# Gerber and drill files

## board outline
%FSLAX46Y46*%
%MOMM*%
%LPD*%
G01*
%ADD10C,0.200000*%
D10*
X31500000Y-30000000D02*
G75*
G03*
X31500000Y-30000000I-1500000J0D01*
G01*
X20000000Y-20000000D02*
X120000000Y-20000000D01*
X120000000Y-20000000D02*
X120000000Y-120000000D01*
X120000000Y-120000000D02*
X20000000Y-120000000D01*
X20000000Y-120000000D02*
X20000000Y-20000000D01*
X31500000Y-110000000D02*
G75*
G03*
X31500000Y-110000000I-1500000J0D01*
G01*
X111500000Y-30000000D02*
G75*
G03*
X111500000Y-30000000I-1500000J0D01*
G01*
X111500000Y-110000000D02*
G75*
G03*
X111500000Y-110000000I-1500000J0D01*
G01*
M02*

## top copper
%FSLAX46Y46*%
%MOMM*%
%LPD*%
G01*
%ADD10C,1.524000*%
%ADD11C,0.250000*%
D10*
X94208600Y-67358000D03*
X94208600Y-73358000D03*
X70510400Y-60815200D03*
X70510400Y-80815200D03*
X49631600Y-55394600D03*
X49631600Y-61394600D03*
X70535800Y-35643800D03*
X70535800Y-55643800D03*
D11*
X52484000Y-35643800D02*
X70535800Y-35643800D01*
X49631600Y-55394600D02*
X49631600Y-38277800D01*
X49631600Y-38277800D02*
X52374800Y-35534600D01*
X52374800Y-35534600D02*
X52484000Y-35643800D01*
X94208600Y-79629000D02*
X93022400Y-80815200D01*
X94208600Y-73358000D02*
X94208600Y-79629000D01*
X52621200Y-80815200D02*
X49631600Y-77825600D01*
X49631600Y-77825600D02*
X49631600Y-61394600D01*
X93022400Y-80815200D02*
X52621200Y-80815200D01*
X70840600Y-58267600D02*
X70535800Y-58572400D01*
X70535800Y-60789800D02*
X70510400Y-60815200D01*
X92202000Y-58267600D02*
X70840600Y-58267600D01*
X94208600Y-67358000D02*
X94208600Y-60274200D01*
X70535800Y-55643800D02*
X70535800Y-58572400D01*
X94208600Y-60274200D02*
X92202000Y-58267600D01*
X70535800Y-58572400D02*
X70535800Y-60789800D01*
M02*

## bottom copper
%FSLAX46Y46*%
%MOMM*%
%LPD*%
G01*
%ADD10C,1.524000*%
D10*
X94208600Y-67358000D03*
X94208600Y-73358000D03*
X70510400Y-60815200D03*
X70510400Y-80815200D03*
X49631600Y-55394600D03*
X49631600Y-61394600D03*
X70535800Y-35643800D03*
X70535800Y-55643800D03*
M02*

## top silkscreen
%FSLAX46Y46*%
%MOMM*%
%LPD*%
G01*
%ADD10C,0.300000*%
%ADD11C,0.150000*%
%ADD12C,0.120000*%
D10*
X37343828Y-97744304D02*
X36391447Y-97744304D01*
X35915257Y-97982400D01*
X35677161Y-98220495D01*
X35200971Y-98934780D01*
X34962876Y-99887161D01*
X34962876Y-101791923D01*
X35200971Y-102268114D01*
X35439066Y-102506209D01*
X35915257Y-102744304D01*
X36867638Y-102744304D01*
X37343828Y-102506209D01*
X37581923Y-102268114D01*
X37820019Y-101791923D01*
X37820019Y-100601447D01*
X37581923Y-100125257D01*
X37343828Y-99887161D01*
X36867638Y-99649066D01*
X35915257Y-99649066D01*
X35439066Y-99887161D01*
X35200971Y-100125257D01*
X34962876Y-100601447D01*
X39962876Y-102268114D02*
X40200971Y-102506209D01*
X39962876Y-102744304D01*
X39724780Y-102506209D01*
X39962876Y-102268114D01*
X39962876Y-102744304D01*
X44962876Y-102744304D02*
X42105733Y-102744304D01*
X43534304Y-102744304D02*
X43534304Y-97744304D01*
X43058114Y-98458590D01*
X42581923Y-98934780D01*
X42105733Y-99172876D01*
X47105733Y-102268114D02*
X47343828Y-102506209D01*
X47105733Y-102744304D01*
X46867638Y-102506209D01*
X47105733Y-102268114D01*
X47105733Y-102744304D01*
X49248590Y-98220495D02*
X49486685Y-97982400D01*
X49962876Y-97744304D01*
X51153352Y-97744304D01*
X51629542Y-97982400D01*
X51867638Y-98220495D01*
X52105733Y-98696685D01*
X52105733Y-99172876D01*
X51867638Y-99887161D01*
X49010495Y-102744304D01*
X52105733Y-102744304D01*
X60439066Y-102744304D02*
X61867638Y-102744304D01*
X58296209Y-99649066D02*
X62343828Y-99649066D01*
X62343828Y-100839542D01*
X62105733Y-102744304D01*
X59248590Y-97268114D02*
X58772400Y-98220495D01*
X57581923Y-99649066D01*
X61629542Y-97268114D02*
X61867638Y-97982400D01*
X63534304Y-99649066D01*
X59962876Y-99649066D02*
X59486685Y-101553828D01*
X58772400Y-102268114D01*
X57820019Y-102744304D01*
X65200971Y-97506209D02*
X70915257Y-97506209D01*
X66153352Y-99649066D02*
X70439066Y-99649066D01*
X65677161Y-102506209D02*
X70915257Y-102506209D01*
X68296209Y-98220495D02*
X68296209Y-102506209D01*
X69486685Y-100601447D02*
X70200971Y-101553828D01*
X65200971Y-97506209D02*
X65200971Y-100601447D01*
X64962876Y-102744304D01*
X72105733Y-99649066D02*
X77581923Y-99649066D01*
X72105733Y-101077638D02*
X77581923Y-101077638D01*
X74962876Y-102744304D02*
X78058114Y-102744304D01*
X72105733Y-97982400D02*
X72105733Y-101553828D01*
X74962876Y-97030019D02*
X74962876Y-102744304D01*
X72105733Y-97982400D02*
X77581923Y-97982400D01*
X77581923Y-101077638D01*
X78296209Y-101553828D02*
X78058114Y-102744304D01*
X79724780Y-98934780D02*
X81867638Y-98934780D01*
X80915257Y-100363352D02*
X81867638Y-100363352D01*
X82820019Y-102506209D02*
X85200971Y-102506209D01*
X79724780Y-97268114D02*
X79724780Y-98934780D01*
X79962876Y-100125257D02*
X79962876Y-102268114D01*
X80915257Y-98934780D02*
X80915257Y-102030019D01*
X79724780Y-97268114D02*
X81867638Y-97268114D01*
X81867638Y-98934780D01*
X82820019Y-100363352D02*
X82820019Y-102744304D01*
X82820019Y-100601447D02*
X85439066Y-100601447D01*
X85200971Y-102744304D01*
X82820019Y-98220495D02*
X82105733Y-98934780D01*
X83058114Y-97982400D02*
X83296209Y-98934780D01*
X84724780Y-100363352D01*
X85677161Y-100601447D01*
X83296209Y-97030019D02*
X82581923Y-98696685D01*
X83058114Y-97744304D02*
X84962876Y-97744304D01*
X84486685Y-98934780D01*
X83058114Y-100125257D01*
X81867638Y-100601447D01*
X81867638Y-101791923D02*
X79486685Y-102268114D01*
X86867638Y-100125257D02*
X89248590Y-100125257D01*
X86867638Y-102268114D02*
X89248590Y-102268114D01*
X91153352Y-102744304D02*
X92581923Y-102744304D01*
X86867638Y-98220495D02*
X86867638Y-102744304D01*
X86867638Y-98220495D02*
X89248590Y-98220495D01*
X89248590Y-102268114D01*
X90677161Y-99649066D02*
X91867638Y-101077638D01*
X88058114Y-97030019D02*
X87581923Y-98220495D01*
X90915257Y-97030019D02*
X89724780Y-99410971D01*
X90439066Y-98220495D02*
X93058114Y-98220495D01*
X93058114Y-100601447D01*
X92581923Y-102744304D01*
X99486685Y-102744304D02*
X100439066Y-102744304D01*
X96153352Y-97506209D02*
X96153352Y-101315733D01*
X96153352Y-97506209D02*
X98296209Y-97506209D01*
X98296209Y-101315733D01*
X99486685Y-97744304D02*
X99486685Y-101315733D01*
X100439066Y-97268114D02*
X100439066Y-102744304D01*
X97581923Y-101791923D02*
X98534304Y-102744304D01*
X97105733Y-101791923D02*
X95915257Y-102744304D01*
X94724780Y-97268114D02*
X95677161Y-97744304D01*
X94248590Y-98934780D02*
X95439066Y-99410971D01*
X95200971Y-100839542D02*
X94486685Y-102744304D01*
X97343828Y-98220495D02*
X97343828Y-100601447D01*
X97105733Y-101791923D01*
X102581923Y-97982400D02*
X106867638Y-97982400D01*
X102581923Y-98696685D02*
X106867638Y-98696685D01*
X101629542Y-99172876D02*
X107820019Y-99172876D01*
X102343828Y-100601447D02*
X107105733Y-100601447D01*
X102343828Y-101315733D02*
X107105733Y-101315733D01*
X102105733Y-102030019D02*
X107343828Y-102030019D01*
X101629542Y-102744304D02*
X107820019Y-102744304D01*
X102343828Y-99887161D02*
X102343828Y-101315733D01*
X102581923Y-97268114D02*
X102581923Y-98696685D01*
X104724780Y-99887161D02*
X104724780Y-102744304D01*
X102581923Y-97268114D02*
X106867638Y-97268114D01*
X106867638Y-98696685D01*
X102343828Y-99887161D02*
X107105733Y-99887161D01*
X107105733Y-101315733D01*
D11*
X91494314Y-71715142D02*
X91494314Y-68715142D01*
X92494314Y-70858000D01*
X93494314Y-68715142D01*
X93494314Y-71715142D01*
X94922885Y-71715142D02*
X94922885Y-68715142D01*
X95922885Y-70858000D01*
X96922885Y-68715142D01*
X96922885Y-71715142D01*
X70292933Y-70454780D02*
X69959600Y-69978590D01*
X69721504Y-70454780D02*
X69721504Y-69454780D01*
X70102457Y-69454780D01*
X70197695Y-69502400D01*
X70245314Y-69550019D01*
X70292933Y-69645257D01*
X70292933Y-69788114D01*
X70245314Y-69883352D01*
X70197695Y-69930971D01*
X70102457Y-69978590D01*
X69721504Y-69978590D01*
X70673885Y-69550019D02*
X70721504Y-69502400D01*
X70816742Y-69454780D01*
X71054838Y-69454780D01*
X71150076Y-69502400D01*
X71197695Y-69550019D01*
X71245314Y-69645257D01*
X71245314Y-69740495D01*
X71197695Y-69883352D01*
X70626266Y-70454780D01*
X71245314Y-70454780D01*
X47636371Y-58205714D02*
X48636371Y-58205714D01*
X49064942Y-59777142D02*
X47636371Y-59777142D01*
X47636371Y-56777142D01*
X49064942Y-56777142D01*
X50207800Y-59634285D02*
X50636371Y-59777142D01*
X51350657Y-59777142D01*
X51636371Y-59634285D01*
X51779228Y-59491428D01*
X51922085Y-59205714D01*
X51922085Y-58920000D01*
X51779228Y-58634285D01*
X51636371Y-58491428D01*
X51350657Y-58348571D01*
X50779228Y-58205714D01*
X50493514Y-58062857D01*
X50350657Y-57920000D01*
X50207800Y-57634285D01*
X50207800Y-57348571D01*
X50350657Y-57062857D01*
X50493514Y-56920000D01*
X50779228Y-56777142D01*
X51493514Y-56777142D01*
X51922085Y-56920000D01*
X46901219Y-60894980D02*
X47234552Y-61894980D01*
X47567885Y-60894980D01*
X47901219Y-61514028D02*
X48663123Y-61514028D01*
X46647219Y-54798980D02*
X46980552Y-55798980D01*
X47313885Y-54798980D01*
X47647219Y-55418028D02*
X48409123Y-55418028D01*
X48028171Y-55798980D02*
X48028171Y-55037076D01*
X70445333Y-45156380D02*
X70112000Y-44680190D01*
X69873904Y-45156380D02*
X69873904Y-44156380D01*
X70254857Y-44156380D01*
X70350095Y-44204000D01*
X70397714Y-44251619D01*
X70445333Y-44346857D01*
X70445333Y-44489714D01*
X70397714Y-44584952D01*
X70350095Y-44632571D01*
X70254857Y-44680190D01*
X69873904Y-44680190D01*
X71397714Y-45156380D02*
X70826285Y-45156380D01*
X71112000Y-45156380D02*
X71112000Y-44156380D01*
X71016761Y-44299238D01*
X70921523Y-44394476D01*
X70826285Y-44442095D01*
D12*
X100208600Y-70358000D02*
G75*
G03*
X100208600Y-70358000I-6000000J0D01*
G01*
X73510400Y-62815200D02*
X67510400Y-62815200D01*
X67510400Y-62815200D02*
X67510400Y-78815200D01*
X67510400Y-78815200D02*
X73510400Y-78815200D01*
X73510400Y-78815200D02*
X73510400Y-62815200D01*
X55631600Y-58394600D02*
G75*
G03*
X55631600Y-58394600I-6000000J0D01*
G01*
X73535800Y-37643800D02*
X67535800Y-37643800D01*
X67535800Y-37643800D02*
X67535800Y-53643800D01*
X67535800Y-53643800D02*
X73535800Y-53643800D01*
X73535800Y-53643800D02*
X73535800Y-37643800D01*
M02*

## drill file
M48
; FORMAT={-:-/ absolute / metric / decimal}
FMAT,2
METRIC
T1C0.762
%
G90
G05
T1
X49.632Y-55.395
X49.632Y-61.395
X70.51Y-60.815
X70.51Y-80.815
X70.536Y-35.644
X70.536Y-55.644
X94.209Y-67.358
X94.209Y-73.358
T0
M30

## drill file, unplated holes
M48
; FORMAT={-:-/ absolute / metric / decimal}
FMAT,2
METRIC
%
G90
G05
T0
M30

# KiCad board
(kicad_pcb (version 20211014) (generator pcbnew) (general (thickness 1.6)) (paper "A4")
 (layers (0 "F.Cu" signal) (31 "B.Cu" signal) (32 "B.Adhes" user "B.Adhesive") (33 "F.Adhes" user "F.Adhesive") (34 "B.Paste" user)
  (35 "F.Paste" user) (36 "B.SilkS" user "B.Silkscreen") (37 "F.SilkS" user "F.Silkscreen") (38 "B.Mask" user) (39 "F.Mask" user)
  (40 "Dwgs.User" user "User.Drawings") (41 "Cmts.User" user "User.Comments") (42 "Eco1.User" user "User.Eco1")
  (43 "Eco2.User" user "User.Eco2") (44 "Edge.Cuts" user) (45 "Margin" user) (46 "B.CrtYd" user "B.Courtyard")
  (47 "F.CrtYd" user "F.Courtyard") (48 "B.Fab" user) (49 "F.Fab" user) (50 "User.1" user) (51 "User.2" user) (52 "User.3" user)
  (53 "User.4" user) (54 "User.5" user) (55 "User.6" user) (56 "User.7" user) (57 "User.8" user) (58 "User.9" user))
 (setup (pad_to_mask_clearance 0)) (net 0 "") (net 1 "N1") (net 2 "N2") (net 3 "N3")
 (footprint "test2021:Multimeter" (layer "F.Cu") (at 94.2086 70.358)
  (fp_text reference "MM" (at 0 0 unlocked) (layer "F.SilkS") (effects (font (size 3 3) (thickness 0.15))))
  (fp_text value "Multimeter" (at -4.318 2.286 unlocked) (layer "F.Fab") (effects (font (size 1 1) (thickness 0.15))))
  (fp_circle (center 0 0) (end 6 0) (layer "F.SilkS") (width 0.12) (fill none))
  (pad "1" thru_hole circle (at 0 -3) (size 1.524 1.524) (drill 0.762) (layers *.Cu *.Mask) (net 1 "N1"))
  (pad "2" thru_hole circle (at 0 3) (size 1.524 1.524) (drill 0.762) (layers *.Cu *.Mask) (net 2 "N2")))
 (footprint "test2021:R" (layer "F.Cu") (at 70.5104 70.8152 -90)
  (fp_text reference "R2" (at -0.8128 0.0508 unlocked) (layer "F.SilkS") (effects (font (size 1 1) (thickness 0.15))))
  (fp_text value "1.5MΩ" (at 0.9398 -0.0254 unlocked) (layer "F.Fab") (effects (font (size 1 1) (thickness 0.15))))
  (fp_rect (start -8 -3) (end 8 3) (layer "F.SilkS") (width 0.12) (fill none))
  (pad "1" thru_hole circle (at -10 0 270) (size 1.524 1.524) (drill 0.762) (layers *.Cu *.Mask) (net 1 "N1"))
  (pad "2" thru_hole circle (at 10 0 270) (size 1.524 1.524) (drill 0.762) (layers *.Cu *.Mask) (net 2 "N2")))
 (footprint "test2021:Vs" (layer "F.Cu") (at 49.6316 58.3946)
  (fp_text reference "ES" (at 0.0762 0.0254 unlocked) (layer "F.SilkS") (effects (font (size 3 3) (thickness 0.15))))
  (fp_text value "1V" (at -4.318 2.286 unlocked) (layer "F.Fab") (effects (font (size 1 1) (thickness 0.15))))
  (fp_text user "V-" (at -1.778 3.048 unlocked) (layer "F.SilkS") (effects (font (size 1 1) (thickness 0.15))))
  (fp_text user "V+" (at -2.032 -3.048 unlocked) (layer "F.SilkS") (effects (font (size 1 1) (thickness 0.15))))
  (fp_circle (center 0 0) (end 6 0) (layer "F.SilkS") (width 0.12) (fill none))
  (pad "1" thru_hole circle (at 0 -3) (size 1.524 1.524) (drill 0.762) (layers *.Cu *.Mask) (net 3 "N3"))
  (pad "2" thru_hole circle (at 0 3) (size 1.524 1.524) (drill 0.762) (layers *.Cu *.Mask) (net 2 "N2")))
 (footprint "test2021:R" (layer "F.Cu") (at 70.5358 45.6438 -90)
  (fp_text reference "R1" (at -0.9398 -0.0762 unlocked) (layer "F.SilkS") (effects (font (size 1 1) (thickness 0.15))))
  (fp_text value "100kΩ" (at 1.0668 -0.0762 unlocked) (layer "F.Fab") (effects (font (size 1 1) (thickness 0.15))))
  (fp_rect (start -8 -3) (end 8 3) (layer "F.SilkS") (width 0.12) (fill none))
  (pad "1" thru_hole circle (at -10 0 270) (size 1.524 1.524) (drill 0.762) (layers *.Cu *.Mask) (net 3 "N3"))
  (pad "2" thru_hole circle (at 10 0 270) (size 1.524 1.524) (drill 0.762) (layers *.Cu *.Mask) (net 1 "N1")))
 (gr_circle (center 30 30) (end 31.5 30) (layer "Edge.Cuts") (width 0.2) (fill none))
 (gr_rect (start 20 20) (end 120 120) (layer "Edge.Cuts") (width 0.2) (fill none))
 (gr_circle (center 30 110) (end 31.5 110) (layer "Edge.Cuts") (width 0.2) (fill none))
 (gr_circle (center 110 30) (end 111.5 30) (layer "Edge.Cuts") (width 0.2) (fill none))
 (gr_circle (center 110 110) (end 111.5 110) (layer "Edge.Cuts") (width 0.2) (fill none))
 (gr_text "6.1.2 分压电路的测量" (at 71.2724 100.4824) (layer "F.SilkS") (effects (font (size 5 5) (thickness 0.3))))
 (segment (start 52.484 35.6438) (end 70.5358 35.6438) (width 0.25) (layer "F.Cu") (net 3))
 (segment (start 49.6316 55.3946) (end 49.6316 38.2778) (width 0.25) (layer "F.Cu") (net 3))
 (segment (start 49.6316 38.2778) (end 52.3748 35.5346) (width 0.25) (layer "F.Cu") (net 3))
 (segment (start 52.3748 35.5346) (end 52.484 35.6438) (width 0.25) (layer "F.Cu") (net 3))
 (segment (start 94.2086 79.629) (end 93.0224 80.8152) (width 0.25) (layer "F.Cu") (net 2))
 (segment (start 94.2086 73.358) (end 94.2086 79.629) (width 0.25) (layer "F.Cu") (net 2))
 (segment (start 52.6212 80.8152) (end 49.6316 77.8256) (width 0.25) (layer "F.Cu") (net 2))
 (segment (start 49.6316 77.8256) (end 49.6316 61.3946) (width 0.25) (layer "F.Cu") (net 2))
 (segment (start 93.0224 80.8152) (end 52.6212 80.8152) (width 0.25) (layer "F.Cu") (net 2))
 (segment (start 70.8406 58.2676) (end 70.5358 58.5724) (width 0.25) (layer "F.Cu") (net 1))
 (segment (start 70.5358 60.7898) (end 70.5104 60.8152) (width 0.25) (layer "F.Cu") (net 1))
 (segment (start 92.202 58.2676) (end 70.8406 58.2676) (width 0.25) (layer "F.Cu") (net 1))
 (segment (start 94.2086 67.358) (end 94.2086 60.2742) (width 0.25) (layer "F.Cu") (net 1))
 (segment (start 70.5358 55.6438) (end 70.5358 58.5724) (width 0.25) (layer "F.Cu") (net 1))
 (segment (start 94.2086 60.2742) (end 92.202 58.2676) (width 0.25) (layer "F.Cu") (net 1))
 (segment (start 70.5358 58.5724) (end 70.5358 60.7898) (width 0.25) (layer "F.Cu") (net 1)))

